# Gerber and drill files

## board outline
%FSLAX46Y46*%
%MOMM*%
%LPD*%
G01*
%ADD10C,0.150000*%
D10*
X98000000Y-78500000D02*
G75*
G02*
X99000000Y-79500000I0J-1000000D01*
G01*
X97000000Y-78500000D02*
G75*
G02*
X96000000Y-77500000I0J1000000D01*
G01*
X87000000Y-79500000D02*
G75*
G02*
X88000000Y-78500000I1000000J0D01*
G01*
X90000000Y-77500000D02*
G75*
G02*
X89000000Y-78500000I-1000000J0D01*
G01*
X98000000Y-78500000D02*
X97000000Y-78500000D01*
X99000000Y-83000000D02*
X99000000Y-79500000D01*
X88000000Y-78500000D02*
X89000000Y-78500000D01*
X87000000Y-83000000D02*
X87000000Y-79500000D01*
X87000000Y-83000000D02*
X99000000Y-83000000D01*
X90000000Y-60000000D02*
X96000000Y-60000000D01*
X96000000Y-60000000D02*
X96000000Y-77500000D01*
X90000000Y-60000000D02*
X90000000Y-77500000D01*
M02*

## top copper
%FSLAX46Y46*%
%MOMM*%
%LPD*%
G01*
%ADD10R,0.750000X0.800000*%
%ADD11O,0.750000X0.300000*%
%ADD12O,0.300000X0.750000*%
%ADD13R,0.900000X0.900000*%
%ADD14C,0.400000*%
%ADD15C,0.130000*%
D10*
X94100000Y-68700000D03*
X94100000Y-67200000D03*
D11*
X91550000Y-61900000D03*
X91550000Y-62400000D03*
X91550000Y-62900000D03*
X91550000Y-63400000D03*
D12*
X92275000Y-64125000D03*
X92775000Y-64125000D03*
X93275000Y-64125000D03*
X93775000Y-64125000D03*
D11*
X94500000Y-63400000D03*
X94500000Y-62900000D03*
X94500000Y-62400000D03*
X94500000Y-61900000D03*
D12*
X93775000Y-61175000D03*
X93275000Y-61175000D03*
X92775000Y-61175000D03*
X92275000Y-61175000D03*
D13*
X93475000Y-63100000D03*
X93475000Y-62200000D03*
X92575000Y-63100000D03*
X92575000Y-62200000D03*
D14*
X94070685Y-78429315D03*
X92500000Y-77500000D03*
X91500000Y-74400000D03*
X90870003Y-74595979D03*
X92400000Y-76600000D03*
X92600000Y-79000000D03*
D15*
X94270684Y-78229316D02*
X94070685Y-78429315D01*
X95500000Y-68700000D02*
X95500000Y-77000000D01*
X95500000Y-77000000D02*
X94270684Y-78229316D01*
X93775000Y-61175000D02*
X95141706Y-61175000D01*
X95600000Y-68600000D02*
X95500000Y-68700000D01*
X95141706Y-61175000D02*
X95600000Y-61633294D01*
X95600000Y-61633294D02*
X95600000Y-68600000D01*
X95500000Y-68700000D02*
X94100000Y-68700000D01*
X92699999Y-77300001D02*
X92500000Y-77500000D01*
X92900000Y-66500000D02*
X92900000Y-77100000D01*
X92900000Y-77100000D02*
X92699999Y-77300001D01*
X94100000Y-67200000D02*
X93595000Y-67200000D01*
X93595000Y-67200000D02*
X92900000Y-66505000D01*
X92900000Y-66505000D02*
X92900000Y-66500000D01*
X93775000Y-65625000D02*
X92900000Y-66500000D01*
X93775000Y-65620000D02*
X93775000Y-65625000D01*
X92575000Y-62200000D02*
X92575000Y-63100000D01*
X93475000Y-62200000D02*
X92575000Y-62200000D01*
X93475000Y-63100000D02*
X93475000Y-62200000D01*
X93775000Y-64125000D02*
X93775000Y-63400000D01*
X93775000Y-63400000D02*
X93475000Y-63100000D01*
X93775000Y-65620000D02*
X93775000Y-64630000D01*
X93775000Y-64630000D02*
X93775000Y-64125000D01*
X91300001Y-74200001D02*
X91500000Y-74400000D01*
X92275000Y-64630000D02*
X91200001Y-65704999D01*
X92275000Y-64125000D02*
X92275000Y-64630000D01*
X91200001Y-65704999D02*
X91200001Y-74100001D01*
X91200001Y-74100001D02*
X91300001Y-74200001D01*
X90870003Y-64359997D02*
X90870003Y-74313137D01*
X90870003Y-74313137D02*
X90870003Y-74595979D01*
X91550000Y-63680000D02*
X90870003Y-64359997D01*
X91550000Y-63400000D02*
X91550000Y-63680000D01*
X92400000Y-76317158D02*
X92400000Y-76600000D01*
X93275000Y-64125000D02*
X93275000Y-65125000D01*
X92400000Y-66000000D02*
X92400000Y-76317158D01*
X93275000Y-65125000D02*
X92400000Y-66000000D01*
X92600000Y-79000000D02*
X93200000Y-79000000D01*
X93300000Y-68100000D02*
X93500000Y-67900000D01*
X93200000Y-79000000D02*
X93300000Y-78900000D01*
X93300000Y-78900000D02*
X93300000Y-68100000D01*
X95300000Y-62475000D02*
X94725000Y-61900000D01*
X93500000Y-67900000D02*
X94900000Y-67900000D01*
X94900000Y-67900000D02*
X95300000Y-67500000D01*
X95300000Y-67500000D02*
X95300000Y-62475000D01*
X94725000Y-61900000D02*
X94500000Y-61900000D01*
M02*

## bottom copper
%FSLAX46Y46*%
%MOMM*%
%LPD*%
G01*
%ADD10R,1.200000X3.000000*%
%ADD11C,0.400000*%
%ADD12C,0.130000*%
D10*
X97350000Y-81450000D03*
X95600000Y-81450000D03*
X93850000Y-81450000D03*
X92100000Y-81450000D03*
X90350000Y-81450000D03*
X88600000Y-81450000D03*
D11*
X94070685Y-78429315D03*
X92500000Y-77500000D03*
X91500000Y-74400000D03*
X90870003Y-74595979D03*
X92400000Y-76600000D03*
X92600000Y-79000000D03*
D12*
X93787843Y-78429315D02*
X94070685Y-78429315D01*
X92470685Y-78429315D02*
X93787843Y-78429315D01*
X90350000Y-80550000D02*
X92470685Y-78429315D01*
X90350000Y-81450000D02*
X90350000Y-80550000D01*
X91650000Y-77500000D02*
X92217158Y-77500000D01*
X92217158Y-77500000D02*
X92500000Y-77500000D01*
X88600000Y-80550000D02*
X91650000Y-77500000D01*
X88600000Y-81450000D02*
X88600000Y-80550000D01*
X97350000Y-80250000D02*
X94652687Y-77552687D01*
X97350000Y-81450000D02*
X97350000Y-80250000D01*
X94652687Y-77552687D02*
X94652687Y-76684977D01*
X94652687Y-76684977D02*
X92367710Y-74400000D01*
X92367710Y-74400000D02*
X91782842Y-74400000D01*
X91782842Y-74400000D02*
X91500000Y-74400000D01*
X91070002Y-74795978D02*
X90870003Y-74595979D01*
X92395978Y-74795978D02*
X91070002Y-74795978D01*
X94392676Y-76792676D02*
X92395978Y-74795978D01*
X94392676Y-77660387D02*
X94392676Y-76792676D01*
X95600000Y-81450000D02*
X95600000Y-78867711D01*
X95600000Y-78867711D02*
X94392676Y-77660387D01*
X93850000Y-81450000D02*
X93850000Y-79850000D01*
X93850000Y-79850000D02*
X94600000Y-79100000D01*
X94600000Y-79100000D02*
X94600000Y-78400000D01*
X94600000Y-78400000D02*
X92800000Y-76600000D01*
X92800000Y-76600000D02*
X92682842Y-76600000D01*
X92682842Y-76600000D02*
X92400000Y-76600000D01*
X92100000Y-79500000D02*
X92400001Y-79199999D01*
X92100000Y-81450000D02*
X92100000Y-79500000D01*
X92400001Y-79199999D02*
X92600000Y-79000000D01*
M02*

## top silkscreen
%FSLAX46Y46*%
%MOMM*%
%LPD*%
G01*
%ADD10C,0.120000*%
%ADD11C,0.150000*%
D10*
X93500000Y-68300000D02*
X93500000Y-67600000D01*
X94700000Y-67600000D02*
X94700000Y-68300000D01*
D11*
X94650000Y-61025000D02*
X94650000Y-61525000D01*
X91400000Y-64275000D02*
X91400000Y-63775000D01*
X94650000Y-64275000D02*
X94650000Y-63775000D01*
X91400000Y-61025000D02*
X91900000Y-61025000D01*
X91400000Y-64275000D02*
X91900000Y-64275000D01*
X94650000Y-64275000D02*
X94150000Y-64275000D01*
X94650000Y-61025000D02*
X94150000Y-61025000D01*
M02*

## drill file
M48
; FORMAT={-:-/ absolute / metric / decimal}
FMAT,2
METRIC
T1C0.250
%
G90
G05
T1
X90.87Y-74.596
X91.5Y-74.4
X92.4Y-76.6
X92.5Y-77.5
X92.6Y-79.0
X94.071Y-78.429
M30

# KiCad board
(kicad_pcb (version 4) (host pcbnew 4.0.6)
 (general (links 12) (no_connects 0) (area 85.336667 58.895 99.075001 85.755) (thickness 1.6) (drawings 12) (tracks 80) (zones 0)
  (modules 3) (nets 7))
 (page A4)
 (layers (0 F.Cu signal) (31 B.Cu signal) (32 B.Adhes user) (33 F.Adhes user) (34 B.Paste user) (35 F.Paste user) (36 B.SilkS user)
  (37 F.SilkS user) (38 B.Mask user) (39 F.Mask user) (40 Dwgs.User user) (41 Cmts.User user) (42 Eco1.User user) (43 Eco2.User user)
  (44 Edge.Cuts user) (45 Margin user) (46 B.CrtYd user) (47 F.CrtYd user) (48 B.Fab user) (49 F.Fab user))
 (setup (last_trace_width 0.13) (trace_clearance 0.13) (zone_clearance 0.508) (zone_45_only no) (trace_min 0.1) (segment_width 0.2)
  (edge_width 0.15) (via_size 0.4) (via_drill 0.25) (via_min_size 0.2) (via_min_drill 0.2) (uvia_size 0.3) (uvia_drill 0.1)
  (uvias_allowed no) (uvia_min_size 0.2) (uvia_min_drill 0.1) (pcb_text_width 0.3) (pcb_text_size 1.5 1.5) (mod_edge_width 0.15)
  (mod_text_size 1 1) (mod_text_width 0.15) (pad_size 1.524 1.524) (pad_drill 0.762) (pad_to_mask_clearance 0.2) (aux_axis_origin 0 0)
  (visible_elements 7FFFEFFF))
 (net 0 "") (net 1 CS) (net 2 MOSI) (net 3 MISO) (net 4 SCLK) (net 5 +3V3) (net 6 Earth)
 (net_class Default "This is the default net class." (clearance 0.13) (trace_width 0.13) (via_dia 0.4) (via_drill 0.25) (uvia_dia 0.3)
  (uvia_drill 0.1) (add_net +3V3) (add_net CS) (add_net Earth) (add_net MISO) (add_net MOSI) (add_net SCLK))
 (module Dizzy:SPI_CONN (layer B.Cu) (at 95.7 78.7 180)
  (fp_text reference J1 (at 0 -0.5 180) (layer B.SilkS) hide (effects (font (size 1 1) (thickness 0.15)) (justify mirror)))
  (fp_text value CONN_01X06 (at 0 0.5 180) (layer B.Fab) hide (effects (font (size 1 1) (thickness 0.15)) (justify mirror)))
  (pad 1 smd rect (at -1.65 -2.75 180) (size 1.2 3) (layers B.Cu B.Paste B.Mask) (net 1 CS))
  (pad 2 smd rect (at 0.1 -2.75 180) (size 1.2 3) (layers B.Cu B.Paste B.Mask) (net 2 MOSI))
  (pad 3 smd rect (at 1.85 -2.75 180) (size 1.2 3) (layers B.Cu B.Paste B.Mask) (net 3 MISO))
  (pad 4 smd rect (at 3.6 -2.75 180) (size 1.2 3) (layers B.Cu B.Paste B.Mask) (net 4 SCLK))
  (pad 5 smd rect (at 5.35 -2.75 180) (size 1.2 3) (layers B.Cu B.Paste B.Mask) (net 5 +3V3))
  (pad 6 smd rect (at 7.1 -2.75 180) (size 1.2 3) (layers B.Cu B.Paste B.Mask) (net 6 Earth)))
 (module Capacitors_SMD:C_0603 (layer F.Cu) (at 94.1 67.95 270)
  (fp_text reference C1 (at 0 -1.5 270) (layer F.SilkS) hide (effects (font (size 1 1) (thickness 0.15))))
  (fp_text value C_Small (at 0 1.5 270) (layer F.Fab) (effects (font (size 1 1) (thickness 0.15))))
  (fp_line (start 0.35 0.6) (end -0.35 0.6) (layer F.SilkS) (width 0.12))
  (fp_line (start -0.35 -0.6) (end 0.35 -0.6) (layer F.SilkS) (width 0.12))
  (pad 2 smd rect (at 0.75 0 270) (size 0.8 0.75) (layers F.Cu F.Paste F.Mask) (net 5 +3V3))
  (pad 1 smd rect (at -0.75 0 270) (size 0.8 0.75) (layers F.Cu F.Paste F.Mask) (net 6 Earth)))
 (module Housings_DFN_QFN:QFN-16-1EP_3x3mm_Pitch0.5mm (layer F.Cu) (at 93.025 62.65)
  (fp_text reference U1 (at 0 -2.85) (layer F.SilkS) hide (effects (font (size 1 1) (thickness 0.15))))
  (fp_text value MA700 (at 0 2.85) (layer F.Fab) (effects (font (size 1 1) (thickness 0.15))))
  (fp_line (start 1.625 -1.625) (end 1.625 -1.125) (layer F.SilkS) (width 0.15))
  (fp_line (start -1.625 1.625) (end -1.625 1.125) (layer F.SilkS) (width 0.15))
  (fp_line (start 1.625 1.625) (end 1.625 1.125) (layer F.SilkS) (width 0.15))
  (fp_line (start -1.625 -1.625) (end -1.125 -1.625) (layer F.SilkS) (width 0.15))
  (fp_line (start -1.625 1.625) (end -1.125 1.625) (layer F.SilkS) (width 0.15))
  (fp_line (start 1.625 1.625) (end 1.125 1.625) (layer F.SilkS) (width 0.15))
  (fp_line (start 1.625 -1.625) (end 1.125 -1.625) (layer F.SilkS) (width 0.15))
  (pad 1 smd oval (at -1.475 -0.75) (size 0.75 0.3) (layers F.Cu F.Paste F.Mask))
  (pad 2 smd oval (at -1.475 -0.25) (size 0.75 0.3) (layers F.Cu F.Paste F.Mask))
  (pad 3 smd oval (at -1.475 0.25) (size 0.75 0.3) (layers F.Cu F.Paste F.Mask))
  (pad 4 smd oval (at -1.475 0.75) (size 0.75 0.3) (layers F.Cu F.Paste F.Mask) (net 2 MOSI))
  (pad 5 smd oval (at -0.75 1.475 90) (size 0.75 0.3) (layers F.Cu F.Paste F.Mask) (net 1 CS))
  (pad 6 smd oval (at -0.25 1.475 90) (size 0.75 0.3) (layers F.Cu F.Paste F.Mask))
  (pad 7 smd oval (at 0.25 1.475 90) (size 0.75 0.3) (layers F.Cu F.Paste F.Mask) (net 3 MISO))
  (pad 8 smd oval (at 0.75 1.475 90) (size 0.75 0.3) (layers F.Cu F.Paste F.Mask) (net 6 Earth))
  (pad 9 smd oval (at 1.475 0.75) (size 0.75 0.3) (layers F.Cu F.Paste F.Mask))
  (pad 10 smd oval (at 1.475 0.25) (size 0.75 0.3) (layers F.Cu F.Paste F.Mask))
  (pad 11 smd oval (at 1.475 -0.25) (size 0.75 0.3) (layers F.Cu F.Paste F.Mask))
  (pad 12 smd oval (at 1.475 -0.75) (size 0.75 0.3) (layers F.Cu F.Paste F.Mask) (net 4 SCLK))
  (pad 13 smd oval (at 0.75 -1.475 90) (size 0.75 0.3) (layers F.Cu F.Paste F.Mask) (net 5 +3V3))
  (pad 14 smd oval (at 0.25 -1.475 90) (size 0.75 0.3) (layers F.Cu F.Paste F.Mask))
  (pad 15 smd oval (at -0.25 -1.475 90) (size 0.75 0.3) (layers F.Cu F.Paste F.Mask))
  (pad 16 smd oval (at -0.75 -1.475 90) (size 0.75 0.3) (layers F.Cu F.Paste F.Mask))
  (pad 17 smd rect (at 0.45 0.45) (size 0.9 0.9) (layers F.Cu F.Paste F.Mask) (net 6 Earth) (solder_paste_margin_ratio -0.2))
  (pad 17 smd rect (at 0.45 -0.45) (size 0.9 0.9) (layers F.Cu F.Paste F.Mask) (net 6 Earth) (solder_paste_margin_ratio -0.2))
  (pad 17 smd rect (at -0.45 0.45) (size 0.9 0.9) (layers F.Cu F.Paste F.Mask) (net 6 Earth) (solder_paste_margin_ratio -0.2))
  (pad 17 smd rect (at -0.45 -0.45) (size 0.9 0.9) (layers F.Cu F.Paste F.Mask) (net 6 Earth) (solder_paste_margin_ratio -0.2)))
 (gr_arc (start 98 79.5) (end 98 78.5) (angle 90) (layer Edge.Cuts) (width 0.15))
 (gr_arc (start 97 77.5) (end 97 78.5) (angle 90) (layer Edge.Cuts) (width 0.15))
 (gr_arc (start 88 79.5) (end 87 79.5) (angle 90) (layer Edge.Cuts) (width 0.15))
 (gr_arc (start 89 77.5) (end 90 77.5) (angle 90) (layer Edge.Cuts) (width 0.15))
 (gr_line (start 98 78.5) (end 97 78.5) (layer Edge.Cuts) (width 0.15))
 (gr_line (start 99 83) (end 99 79.5) (layer Edge.Cuts) (width 0.15))
 (gr_line (start 88 78.5) (end 89 78.5) (layer Edge.Cuts) (width 0.15))
 (gr_line (start 87 83) (end 87 79.5) (layer Edge.Cuts) (width 0.15))
 (gr_line (start 87 83) (end 99 83) (layer Edge.Cuts) (width 0.15))
 (gr_line (start 90 60) (end 96 60) (layer Edge.Cuts) (width 0.15))
 (gr_line (start 96 60) (end 96 77.5) (layer Edge.Cuts) (width 0.15))
 (gr_line (start 90 60) (end 90 77.5) (layer Edge.Cuts) (width 0.15))
 (segment (start 94.270684 78.229316) (end 94.070685 78.429315) (width 0.13) (layer F.Cu) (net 5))
 (segment (start 95.5 68.7) (end 95.5 77) (width 0.13) (layer F.Cu) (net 5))
 (segment (start 93.787843 78.429315) (end 94.070685 78.429315) (width 0.13) (layer B.Cu) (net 5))
 (segment (start 92.470685 78.429315) (end 93.787843 78.429315) (width 0.13) (layer B.Cu) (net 5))
 (segment (start 90.35 80.55) (end 92.470685 78.429315) (width 0.13) (layer B.Cu) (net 5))
 (segment (start 95.5 77) (end 94.270684 78.229316) (width 0.13) (layer F.Cu) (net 5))
 (segment (start 90.35 81.45) (end 90.35 80.55) (width 0.13) (layer B.Cu) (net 5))
 (via (at 94.070685 78.429315) (size 0.4) (drill 0.25) (layers F.Cu B.Cu) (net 5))
 (segment (start 93.775 61.175) (end 95.141706 61.175) (width 0.13) (layer F.Cu) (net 5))
 (segment (start 95.6 68.6) (end 95.5 68.7) (width 0.13) (layer F.Cu) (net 5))
 (segment (start 95.141706 61.175) (end 95.6 61.633294) (width 0.13) (layer F.Cu) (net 5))
 (segment (start 95.6 61.633294) (end 95.6 68.6) (width 0.13) (layer F.Cu) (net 5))
 (segment (start 95.5 68.7) (end 94.1 68.7) (width 0.13) (layer F.Cu) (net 5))
 (segment (start 91.65 77.5) (end 92.217158 77.5) (width 0.13) (layer B.Cu) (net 6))
 (segment (start 92.217158 77.5) (end 92.5 77.5) (width 0.13) (layer B.Cu) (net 6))
 (segment (start 88.6 80.55) (end 91.65 77.5) (width 0.13) (layer B.Cu) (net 6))
 (segment (start 88.6 81.45) (end 88.6 80.55) (width 0.13) (layer B.Cu) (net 6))
 (segment (start 92.699999 77.300001) (end 92.5 77.5) (width 0.13) (layer F.Cu) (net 6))
 (segment (start 92.9 66.5) (end 92.9 77.1) (width 0.13) (layer F.Cu) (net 6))
 (segment (start 92.9 77.1) (end 92.699999 77.300001) (width 0.13) (layer F.Cu) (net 6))
 (via (at 92.5 77.5) (size 0.4) (drill 0.25) (layers F.Cu B.Cu) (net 6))
 (segment (start 94.1 67.2) (end 93.595 67.2) (width 0.13) (layer F.Cu) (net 6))
 (segment (start 93.595 67.2) (end 92.9 66.505) (width 0.13) (layer F.Cu) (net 6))
 (segment (start 92.9 66.505) (end 92.9 66.5) (width 0.13) (layer F.Cu) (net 6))
 (segment (start 93.775 65.625) (end 92.9 66.5) (width 0.13) (layer F.Cu) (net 6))
 (segment (start 93.775 65.62) (end 93.775 65.625) (width 0.13) (layer F.Cu) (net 6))
 (segment (start 92.575 62.2) (end 92.575 63.1) (width 0.13) (layer F.Cu) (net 6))
 (segment (start 93.475 62.2) (end 92.575 62.2) (width 0.13) (layer F.Cu) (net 6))
 (segment (start 93.475 63.1) (end 93.475 62.2) (width 0.13) (layer F.Cu) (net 6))
 (segment (start 93.775 64.125) (end 93.775 63.4) (width 0.13) (layer F.Cu) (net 6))
 (segment (start 93.775 63.4) (end 93.475 63.1) (width 0.13) (layer F.Cu) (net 6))
 (segment (start 93.775 65.62) (end 93.775 64.63) (width 0.13) (layer F.Cu) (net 6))
 (segment (start 93.775 64.63) (end 93.775 64.125) (width 0.13) (layer F.Cu) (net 6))
 (segment (start 97.35 80.25) (end 94.652687 77.552687) (width 0.13) (layer B.Cu) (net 1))
 (segment (start 97.35 81.45) (end 97.35 80.25) (width 0.13) (layer B.Cu) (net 1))
 (segment (start 94.652687 77.552687) (end 94.652687 76.684977) (width 0.13) (layer B.Cu) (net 1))
 (segment (start 94.652687 76.684977) (end 92.36771 74.4) (width 0.13) (layer B.Cu) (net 1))
 (segment (start 92.36771 74.4) (end 91.782842 74.4) (width 0.13) (layer B.Cu) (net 1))
 (segment (start 91.782842 74.4) (end 91.5 74.4) (width 0.13) (layer B.Cu) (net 1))
 (segment (start 91.300001 74.200001) (end 91.5 74.4) (width 0.13) (layer F.Cu) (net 1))
 (segment (start 92.275 64.63) (end 91.200001 65.704999) (width 0.13) (layer F.Cu) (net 1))
 (segment (start 92.275 64.125) (end 92.275 64.63) (width 0.13) (layer F.Cu) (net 1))
 (segment (start 91.200001 65.704999) (end 91.200001 74.100001) (width 0.13) (layer F.Cu) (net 1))
 (via (at 91.5 74.4) (size 0.4) (drill 0.25) (layers F.Cu B.Cu) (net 1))
 (segment (start 91.200001 74.100001) (end 91.300001 74.200001) (width 0.13) (layer F.Cu) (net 1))
 (segment (start 91.070002 74.795978) (end 90.870003 74.595979) (width 0.13) (layer B.Cu) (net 2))
 (segment (start 92.395978 74.795978) (end 91.070002 74.795978) (width 0.13) (layer B.Cu) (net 2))
 (segment (start 94.392676 76.792676) (end 92.395978 74.795978) (width 0.13) (layer B.Cu) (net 2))
 (segment (start 94.392676 77.660387) (end 94.392676 76.792676) (width 0.13) (layer B.Cu) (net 2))
 (segment (start 95.6 81.45) (end 95.6 78.867711) (width 0.13) (layer B.Cu) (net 2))
 (segment (start 95.6 78.867711) (end 94.392676 77.660387) (width 0.13) (layer B.Cu) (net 2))
 (segment (start 90.870003 64.359997) (end 90.870003 74.313137) (width 0.13) (layer F.Cu) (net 2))
 (segment (start 90.870003 74.313137) (end 90.870003 74.595979) (width 0.13) (layer F.Cu) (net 2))
 (via (at 90.870003 74.595979) (size 0.4) (drill 0.25) (layers F.Cu B.Cu) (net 2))
 (segment (start 91.55 63.68) (end 90.870003 64.359997) (width 0.13) (layer F.Cu) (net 2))
 (segment (start 91.55 63.4) (end 91.55 63.68) (width 0.13) (layer F.Cu) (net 2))
 (segment (start 93.85 81.45) (end 93.85 79.85) (width 0.13) (layer B.Cu) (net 3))
 (segment (start 93.85 79.85) (end 94.6 79.1) (width 0.13) (layer B.Cu) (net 3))
 (segment (start 94.6 79.1) (end 94.6 78.4) (width 0.13) (layer B.Cu) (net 3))
 (segment (start 94.6 78.4) (end 92.8 76.6) (width 0.13) (layer B.Cu) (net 3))
 (segment (start 92.8 76.6) (end 92.682842 76.6) (width 0.13) (layer B.Cu) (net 3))
 (segment (start 92.682842 76.6) (end 92.4 76.6) (width 0.13) (layer B.Cu) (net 3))
 (via (at 92.4 76.6) (size 0.4) (drill 0.25) (layers F.Cu B.Cu) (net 3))
 (segment (start 92.4 76.317158) (end 92.4 76.6) (width 0.13) (layer F.Cu) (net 3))
 (segment (start 93.275 64.125) (end 93.275 65.125) (width 0.13) (layer F.Cu) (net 3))
 (segment (start 92.4 66) (end 92.4 76.317158) (width 0.13) (layer F.Cu) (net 3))
 (segment (start 93.275 65.125) (end 92.4 66) (width 0.13) (layer F.Cu) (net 3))
 (segment (start 92.6 79) (end 93.2 79) (width 0.13) (layer F.Cu) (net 4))
 (segment (start 93.3 68.1) (end 93.5 67.9) (width 0.13) (layer F.Cu) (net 4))
 (segment (start 93.2 79) (end 93.3 78.9) (width 0.13) (layer F.Cu) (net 4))
 (segment (start 93.3 78.9) (end 93.3 68.1) (width 0.13) (layer F.Cu) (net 4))
 (segment (start 95.3 62.475) (end 94.725 61.9) (width 0.13) (layer F.Cu) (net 4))
 (segment (start 93.5 67.9) (end 94.9 67.9) (width 0.13) (layer F.Cu) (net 4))
 (segment (start 94.9 67.9) (end 95.3 67.5) (width 0.13) (layer F.Cu) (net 4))
 (segment (start 95.3 67.5) (end 95.3 62.475) (width 0.13) (layer F.Cu) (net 4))
 (segment (start 94.725 61.9) (end 94.5 61.9) (width 0.13) (layer F.Cu) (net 4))
 (segment (start 92.1 79.5) (end 92.400001 79.199999) (width 0.13) (layer B.Cu) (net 4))
 (segment (start 92.1 81.45) (end 92.1 79.5) (width 0.13) (layer B.Cu) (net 4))
 (segment (start 92.400001 79.199999) (end 92.6 79) (width 0.13) (layer B.Cu) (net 4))
 (via (at 92.6 79) (size 0.4) (drill 0.25) (layers F.Cu B.Cu) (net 4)))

